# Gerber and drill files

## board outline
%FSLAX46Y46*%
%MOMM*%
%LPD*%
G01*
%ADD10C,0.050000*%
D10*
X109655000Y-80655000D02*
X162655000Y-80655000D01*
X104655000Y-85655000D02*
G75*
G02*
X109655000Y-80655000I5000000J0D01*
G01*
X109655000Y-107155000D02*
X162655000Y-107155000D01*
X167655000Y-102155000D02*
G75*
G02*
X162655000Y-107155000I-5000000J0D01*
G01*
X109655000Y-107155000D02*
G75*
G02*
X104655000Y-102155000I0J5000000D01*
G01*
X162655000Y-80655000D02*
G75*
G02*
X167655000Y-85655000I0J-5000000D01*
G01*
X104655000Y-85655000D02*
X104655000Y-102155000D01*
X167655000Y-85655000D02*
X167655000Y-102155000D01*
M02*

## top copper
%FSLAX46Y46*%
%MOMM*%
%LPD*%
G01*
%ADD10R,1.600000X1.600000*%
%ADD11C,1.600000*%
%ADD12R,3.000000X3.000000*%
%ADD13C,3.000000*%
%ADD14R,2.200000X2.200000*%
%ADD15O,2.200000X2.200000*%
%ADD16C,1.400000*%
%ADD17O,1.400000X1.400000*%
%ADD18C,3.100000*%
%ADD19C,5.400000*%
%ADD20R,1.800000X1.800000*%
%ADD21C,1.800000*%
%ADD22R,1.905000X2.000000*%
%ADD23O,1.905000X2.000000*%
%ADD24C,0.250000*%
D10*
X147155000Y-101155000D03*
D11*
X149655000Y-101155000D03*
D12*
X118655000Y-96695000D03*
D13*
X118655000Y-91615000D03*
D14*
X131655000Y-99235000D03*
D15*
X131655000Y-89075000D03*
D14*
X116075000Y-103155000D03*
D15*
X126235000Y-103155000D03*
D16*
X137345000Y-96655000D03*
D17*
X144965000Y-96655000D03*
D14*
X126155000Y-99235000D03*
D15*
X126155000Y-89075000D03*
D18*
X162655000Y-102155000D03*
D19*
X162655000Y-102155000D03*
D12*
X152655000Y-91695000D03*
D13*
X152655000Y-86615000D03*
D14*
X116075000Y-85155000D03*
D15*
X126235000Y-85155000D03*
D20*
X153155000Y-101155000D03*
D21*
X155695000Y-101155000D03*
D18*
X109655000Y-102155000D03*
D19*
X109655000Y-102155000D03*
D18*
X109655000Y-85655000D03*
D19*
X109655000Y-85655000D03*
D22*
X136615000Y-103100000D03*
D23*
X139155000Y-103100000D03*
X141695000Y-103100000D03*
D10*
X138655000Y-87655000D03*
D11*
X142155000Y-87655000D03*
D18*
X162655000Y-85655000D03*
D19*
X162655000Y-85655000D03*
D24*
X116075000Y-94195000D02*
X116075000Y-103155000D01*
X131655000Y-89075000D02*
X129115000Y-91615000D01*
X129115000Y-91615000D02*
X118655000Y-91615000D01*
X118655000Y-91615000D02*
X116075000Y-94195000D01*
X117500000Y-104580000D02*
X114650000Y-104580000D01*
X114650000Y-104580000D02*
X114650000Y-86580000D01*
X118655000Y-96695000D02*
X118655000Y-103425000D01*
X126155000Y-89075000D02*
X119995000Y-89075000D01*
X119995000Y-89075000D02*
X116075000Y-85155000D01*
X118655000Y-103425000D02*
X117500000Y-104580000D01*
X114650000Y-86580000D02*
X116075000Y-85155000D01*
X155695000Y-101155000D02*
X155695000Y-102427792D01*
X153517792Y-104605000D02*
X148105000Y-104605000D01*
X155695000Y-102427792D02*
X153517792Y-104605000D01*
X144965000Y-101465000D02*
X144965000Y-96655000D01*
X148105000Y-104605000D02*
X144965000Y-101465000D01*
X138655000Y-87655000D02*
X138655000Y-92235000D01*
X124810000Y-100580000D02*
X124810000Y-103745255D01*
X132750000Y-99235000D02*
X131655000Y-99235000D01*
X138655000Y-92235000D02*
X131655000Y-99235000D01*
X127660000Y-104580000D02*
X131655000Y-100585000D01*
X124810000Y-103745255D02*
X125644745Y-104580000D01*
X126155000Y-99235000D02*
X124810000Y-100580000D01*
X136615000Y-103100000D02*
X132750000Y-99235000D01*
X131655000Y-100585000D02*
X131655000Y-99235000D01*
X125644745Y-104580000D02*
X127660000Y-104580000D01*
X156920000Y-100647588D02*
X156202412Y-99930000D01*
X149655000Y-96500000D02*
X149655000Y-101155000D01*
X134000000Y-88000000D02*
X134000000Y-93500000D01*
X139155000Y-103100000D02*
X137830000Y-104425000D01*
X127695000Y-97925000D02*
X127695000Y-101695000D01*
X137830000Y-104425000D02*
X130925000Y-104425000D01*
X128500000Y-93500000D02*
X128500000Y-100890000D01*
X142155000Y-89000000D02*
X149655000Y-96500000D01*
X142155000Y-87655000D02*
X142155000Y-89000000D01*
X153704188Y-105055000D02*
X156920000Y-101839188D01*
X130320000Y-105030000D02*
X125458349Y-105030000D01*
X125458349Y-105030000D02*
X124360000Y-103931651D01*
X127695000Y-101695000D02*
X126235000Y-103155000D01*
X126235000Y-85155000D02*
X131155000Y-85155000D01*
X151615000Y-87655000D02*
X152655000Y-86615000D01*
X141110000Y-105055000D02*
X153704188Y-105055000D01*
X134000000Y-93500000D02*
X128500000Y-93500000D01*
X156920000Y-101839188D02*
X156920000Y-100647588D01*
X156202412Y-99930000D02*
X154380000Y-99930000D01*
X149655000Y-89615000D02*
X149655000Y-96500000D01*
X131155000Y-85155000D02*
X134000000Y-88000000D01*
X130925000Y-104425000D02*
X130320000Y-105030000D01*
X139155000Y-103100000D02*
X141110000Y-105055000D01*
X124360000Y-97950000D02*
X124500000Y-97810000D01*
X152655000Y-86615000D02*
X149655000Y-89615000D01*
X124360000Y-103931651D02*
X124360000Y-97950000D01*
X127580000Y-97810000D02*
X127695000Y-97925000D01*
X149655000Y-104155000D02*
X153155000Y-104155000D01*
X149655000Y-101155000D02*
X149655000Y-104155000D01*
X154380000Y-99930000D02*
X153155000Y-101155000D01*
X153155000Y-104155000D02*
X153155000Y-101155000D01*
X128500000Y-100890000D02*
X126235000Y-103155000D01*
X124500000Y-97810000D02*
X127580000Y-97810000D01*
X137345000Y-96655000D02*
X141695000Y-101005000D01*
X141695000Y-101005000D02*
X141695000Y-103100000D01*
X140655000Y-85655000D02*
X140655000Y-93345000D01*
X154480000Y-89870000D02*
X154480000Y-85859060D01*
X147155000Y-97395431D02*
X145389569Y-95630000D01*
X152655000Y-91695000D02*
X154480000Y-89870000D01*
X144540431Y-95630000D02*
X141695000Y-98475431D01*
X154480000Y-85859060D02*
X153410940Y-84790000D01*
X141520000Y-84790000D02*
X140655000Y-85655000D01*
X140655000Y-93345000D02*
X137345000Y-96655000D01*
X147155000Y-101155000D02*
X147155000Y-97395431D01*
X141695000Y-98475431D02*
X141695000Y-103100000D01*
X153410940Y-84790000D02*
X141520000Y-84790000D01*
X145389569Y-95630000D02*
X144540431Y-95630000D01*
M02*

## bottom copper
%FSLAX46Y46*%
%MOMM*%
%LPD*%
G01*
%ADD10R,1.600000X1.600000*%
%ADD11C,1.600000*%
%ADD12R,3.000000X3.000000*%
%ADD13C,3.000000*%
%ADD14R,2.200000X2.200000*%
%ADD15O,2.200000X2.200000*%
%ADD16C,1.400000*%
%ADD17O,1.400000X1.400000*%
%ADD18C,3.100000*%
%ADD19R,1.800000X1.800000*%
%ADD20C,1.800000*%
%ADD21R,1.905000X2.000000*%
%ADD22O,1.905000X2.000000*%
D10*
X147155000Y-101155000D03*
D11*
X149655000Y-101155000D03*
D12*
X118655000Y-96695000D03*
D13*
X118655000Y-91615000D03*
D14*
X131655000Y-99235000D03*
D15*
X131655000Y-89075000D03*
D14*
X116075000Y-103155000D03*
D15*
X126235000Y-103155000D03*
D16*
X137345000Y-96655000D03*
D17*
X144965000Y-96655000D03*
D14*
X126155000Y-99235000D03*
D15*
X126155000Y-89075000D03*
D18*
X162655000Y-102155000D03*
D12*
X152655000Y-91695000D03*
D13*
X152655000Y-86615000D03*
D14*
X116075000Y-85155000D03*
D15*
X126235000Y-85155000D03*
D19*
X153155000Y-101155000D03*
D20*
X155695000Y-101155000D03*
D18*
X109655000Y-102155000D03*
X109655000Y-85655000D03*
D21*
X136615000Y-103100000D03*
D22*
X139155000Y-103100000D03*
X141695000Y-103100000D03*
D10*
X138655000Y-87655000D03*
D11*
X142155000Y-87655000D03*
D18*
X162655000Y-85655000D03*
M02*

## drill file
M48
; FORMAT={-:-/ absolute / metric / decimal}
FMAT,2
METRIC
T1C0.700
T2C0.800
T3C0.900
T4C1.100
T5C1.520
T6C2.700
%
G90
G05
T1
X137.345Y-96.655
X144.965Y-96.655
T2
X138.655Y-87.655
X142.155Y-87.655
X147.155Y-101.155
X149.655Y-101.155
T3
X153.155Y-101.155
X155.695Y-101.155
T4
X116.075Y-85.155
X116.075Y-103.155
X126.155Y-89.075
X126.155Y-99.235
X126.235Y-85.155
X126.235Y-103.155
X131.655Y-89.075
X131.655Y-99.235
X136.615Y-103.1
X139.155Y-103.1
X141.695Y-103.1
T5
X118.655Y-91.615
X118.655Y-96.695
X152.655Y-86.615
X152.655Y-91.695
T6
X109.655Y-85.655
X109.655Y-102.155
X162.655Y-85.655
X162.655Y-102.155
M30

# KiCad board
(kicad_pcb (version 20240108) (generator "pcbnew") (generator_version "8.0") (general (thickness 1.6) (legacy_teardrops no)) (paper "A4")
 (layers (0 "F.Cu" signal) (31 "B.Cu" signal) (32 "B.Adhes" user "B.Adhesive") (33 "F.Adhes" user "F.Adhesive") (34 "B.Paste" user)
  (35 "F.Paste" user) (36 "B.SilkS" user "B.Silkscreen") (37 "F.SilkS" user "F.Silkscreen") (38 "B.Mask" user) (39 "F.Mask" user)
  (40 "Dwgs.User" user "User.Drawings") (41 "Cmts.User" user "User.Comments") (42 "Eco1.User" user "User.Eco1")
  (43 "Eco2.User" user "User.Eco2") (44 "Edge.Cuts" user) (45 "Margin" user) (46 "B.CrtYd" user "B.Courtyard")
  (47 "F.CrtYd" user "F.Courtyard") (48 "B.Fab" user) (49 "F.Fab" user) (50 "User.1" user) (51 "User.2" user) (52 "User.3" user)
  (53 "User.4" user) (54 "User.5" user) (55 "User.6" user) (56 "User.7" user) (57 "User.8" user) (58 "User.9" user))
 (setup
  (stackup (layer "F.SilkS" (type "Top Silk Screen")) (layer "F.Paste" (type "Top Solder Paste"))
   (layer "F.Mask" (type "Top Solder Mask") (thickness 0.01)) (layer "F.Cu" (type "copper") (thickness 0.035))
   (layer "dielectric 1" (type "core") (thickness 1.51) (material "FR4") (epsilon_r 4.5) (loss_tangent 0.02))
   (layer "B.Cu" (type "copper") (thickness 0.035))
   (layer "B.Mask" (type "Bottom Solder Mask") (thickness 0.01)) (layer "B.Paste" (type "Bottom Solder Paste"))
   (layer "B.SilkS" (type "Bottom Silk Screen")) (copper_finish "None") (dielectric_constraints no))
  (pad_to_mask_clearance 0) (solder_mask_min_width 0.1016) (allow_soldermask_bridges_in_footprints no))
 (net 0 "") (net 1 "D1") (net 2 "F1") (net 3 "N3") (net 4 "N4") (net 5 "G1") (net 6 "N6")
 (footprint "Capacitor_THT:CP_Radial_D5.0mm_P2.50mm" (layer "F.Cu") (at 147.155 101.155)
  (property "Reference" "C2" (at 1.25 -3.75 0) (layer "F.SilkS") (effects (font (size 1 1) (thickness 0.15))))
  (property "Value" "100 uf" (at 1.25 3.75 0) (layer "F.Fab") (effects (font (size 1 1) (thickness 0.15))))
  (pad "1" thru_hole rect (at 0 0) (size 1.6 1.6) (drill 0.8) (layers "*.Cu" "*.Mask") (remove_unused_layers no) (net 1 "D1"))
  (pad "2" thru_hole circle (at 2.5 0) (size 1.6 1.6) (drill 0.8) (layers "*.Cu" "*.Mask") (remove_unused_layers no) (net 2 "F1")))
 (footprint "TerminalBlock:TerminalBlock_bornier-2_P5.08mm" (layer "F.Cu") (at 118.655 96.695 90)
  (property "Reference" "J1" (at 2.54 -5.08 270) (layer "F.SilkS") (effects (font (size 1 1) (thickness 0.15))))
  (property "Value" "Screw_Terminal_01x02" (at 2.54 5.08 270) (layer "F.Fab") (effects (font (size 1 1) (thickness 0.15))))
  (pad "1" thru_hole rect (at 0 0 90) (size 3 3) (drill 1.52) (layers "*.Cu" "*.Mask") (remove_unused_layers no) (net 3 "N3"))
  (pad "2" thru_hole circle (at 5.08 0 90) (size 3 3) (drill 1.52) (layers "*.Cu" "*.Mask") (remove_unused_layers no) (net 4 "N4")))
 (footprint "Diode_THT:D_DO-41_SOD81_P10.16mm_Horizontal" (layer "F.Cu") (at 131.655 99.235 90)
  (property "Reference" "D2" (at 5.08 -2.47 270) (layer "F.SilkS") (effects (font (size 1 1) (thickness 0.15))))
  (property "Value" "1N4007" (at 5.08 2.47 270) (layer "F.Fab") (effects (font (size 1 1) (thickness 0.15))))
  (pad "1" thru_hole rect (at 0 0 90) (size 2.2 2.2) (drill 1.1) (layers "*.Cu" "*.Mask") (remove_unused_layers no) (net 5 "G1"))
  (pad "2" thru_hole oval (at 10.16 0 90) (size 2.2 2.2) (drill 1.1) (layers "*.Cu" "*.Mask") (remove_unused_layers no) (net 4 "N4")))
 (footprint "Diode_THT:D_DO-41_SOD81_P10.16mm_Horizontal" (layer "F.Cu") (at 116.075 103.155)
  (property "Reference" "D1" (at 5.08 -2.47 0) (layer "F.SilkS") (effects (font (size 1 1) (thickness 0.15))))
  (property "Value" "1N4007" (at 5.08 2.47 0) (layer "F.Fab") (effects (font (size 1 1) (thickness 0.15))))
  (pad "1" thru_hole rect (at 0 0) (size 2.2 2.2) (drill 1.1) (layers "*.Cu" "*.Mask") (remove_unused_layers no) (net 4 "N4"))
  (pad "2" thru_hole oval (at 10.16 0) (size 2.2 2.2) (drill 1.1) (layers "*.Cu" "*.Mask") (remove_unused_layers no) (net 2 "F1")))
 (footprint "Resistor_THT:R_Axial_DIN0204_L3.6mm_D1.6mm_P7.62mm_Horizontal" (layer "F.Cu") (at 137.345 96.655)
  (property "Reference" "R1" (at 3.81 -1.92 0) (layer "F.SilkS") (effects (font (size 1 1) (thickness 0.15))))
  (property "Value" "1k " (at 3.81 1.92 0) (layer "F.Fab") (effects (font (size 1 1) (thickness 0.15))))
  (pad "1" thru_hole circle (at 0 0) (size 1.4 1.4) (drill 0.7) (layers "*.Cu" "*.Mask") (remove_unused_layers no) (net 1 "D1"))
  (pad "2" thru_hole oval (at 7.62 0) (size 1.4 1.4) (drill 0.7) (layers "*.Cu" "*.Mask") (remove_unused_layers no) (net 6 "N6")))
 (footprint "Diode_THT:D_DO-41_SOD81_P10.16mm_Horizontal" (layer "F.Cu") (at 126.155 99.235 90)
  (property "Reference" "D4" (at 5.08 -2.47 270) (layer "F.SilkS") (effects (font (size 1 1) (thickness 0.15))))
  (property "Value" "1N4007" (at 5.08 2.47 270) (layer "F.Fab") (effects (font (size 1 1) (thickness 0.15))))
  (pad "1" thru_hole rect (at 0 0 90) (size 2.2 2.2) (drill 1.1) (layers "*.Cu" "*.Mask") (remove_unused_layers no) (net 5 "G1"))
  (pad "2" thru_hole oval (at 10.16 0 90) (size 2.2 2.2) (drill 1.1) (layers "*.Cu" "*.Mask") (remove_unused_layers no) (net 3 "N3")))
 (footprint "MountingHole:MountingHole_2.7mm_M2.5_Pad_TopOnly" (layer "F.Cu") (at 162.655 102.155)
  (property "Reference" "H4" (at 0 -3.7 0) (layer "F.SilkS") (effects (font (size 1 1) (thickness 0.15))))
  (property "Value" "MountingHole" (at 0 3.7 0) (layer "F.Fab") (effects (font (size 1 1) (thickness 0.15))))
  (pad "1" thru_hole circle (at 0 0) (size 3.1 3.1) (drill 2.7) (layers "*.Cu" "*.Mask") (remove_unused_layers no))
  (pad "1" connect circle (at 0 0) (size 5.4 5.4) (layers "F.Cu" "F.Mask")))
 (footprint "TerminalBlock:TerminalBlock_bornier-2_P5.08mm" (layer "F.Cu") (at 152.655 91.695 90)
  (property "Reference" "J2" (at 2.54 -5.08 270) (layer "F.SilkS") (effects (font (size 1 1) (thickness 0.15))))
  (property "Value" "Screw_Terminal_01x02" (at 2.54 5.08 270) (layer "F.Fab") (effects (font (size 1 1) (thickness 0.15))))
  (pad "1" thru_hole rect (at 0 0 90) (size 3 3) (drill 1.52) (layers "*.Cu" "*.Mask") (remove_unused_layers no) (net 1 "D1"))
  (pad "2" thru_hole circle (at 5.08 0 90) (size 3 3) (drill 1.52) (layers "*.Cu" "*.Mask") (remove_unused_layers no) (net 2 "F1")))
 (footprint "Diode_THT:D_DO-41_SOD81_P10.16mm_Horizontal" (layer "F.Cu") (at 116.075 85.155)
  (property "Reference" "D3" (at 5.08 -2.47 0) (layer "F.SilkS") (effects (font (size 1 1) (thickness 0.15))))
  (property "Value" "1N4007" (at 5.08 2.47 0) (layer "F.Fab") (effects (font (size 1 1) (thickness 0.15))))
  (pad "1" thru_hole rect (at 0 0) (size 2.2 2.2) (drill 1.1) (layers "*.Cu" "*.Mask") (remove_unused_layers no) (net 3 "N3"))
  (pad "2" thru_hole oval (at 10.16 0) (size 2.2 2.2) (drill 1.1) (layers "*.Cu" "*.Mask") (remove_unused_layers no) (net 2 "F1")))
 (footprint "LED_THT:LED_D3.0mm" (layer "F.Cu") (at 153.155 101.155)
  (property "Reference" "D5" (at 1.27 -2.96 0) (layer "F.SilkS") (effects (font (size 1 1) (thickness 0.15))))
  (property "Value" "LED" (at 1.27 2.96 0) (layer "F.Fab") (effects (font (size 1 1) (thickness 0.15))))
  (pad "1" thru_hole rect (at 0 0) (size 1.8 1.8) (drill 0.9) (layers "*.Cu" "*.Mask") (remove_unused_layers no) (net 2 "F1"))
  (pad "2" thru_hole circle (at 2.54 0) (size 1.8 1.8) (drill 0.9) (layers "*.Cu" "*.Mask") (remove_unused_layers no) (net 6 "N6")))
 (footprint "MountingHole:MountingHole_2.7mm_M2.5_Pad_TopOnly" (layer "F.Cu") (at 109.655 102.155)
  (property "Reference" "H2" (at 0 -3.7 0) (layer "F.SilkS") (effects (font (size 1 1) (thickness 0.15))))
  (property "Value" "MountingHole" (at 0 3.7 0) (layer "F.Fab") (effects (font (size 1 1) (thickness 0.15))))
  (pad "1" thru_hole circle (at 0 0) (size 3.1 3.1) (drill 2.7) (layers "*.Cu" "*.Mask") (remove_unused_layers no))
  (pad "1" connect circle (at 0 0) (size 5.4 5.4) (layers "F.Cu" "F.Mask")))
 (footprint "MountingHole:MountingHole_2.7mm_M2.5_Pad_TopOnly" (layer "F.Cu") (at 109.655 85.655)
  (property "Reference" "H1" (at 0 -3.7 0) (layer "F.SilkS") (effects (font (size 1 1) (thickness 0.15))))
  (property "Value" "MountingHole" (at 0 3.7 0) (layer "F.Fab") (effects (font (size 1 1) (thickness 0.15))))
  (pad "1" thru_hole circle (at 0 0) (size 3.1 3.1) (drill 2.7) (layers "*.Cu" "*.Mask") (remove_unused_layers no))
  (pad "1" connect circle (at 0 0) (size 5.4 5.4) (layers "F.Cu" "F.Mask")))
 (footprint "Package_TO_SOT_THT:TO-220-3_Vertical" (layer "F.Cu") (at 136.615 103.1)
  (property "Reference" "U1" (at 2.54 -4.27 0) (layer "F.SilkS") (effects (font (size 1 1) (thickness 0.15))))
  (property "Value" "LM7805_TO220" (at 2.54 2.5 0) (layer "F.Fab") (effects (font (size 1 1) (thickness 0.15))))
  (pad "1" thru_hole rect (at 0 0) (size 1.905 2) (drill 1.1) (layers "*.Cu" "*.Mask") (remove_unused_layers no) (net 5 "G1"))
  (pad "2" thru_hole oval (at 2.54 0) (size 1.905 2) (drill 1.1) (layers "*.Cu" "*.Mask") (remove_unused_layers no) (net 2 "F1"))
  (pad "3" thru_hole oval (at 5.08 0) (size 1.905 2) (drill 1.1) (layers "*.Cu" "*.Mask") (remove_unused_layers no) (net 1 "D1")))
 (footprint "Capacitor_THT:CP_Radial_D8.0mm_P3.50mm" (layer "F.Cu") (at 138.655 87.655)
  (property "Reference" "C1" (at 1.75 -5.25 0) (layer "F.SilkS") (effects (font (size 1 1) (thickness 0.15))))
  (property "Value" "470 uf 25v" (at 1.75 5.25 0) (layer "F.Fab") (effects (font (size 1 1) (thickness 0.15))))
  (pad "1" thru_hole rect (at 0 0) (size 1.6 1.6) (drill 0.8) (layers "*.Cu" "*.Mask") (remove_unused_layers no) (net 5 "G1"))
  (pad "2" thru_hole circle (at 3.5 0) (size 1.6 1.6) (drill 0.8) (layers "*.Cu" "*.Mask") (remove_unused_layers no) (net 2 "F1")))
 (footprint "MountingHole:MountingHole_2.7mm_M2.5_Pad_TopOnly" (layer "F.Cu") (at 162.655 85.655)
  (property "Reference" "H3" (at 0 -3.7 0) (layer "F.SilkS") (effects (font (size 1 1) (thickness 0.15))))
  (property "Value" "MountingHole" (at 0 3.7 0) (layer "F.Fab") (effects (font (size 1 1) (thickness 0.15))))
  (pad "1" thru_hole circle (at 0 0) (size 3.1 3.1) (drill 2.7) (layers "*.Cu" "*.Mask") (remove_unused_layers no))
  (pad "1" connect circle (at 0 0) (size 5.4 5.4) (layers "F.Cu" "F.Mask")))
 (gr_line (start 109.655 80.655) (end 162.655 80.655) (stroke (width 0.05) (type default)) (layer "Edge.Cuts"))
 (gr_arc (start 104.655 85.655) (mid 106.119466 82.119466) (end 109.655 80.655) (stroke (width 0.05) (type default)) (layer "Edge.Cuts"))
 (gr_line (start 109.655 107.155) (end 162.655 107.155) (stroke (width 0.05) (type default)) (layer "Edge.Cuts"))
 (gr_arc (start 167.655 102.155) (mid 166.190534 105.690534) (end 162.655 107.155) (stroke (width 0.05) (type default)) (layer "Edge.Cuts"))
 (gr_arc (start 109.655 107.155) (mid 106.119466 105.690534) (end 104.655 102.155) (stroke (width 0.05) (type default)) (layer "Edge.Cuts"))
 (gr_arc (start 162.655 80.655) (mid 166.190534 82.119466) (end 167.655 85.655) (stroke (width 0.05) (type default)) (layer "Edge.Cuts"))
 (gr_line (start 104.655 85.655) (end 104.655 102.155) (stroke (width 0.05) (type default)) (layer "Edge.Cuts"))
 (gr_line (start 167.655 85.655) (end 167.655 102.155) (stroke (width 0.05) (type default)) (layer "Edge.Cuts"))
 (segment (start 116.075 94.195) (end 116.075 103.155) (width 0.25) (layer "F.Cu") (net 4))
 (segment (start 131.655 89.075) (end 129.115 91.615) (width 0.25) (layer "F.Cu") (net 4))
 (segment (start 129.115 91.615) (end 118.655 91.615) (width 0.25) (layer "F.Cu") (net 4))
 (segment (start 118.655 91.615) (end 116.075 94.195) (width 0.25) (layer "F.Cu") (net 4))
 (segment (start 117.5 104.58) (end 114.65 104.58) (width 0.25) (layer "F.Cu") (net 3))
 (segment (start 114.65 104.58) (end 114.65 86.58) (width 0.25) (layer "F.Cu") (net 3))
 (segment (start 118.655 96.695) (end 118.655 103.425) (width 0.25) (layer "F.Cu") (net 3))
 (segment (start 126.155 89.075) (end 119.995 89.075) (width 0.25) (layer "F.Cu") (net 3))
 (segment (start 119.995 89.075) (end 116.075 85.155) (width 0.25) (layer "F.Cu") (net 3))
 (segment (start 118.655 103.425) (end 117.5 104.58) (width 0.25) (layer "F.Cu") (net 3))
 (segment (start 114.65 86.58) (end 116.075 85.155) (width 0.25) (layer "F.Cu") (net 3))
 (segment (start 155.695 101.155) (end 155.695 102.427792) (width 0.25) (layer "F.Cu") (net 6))
 (segment (start 153.517792 104.605) (end 148.105 104.605) (width 0.25) (layer "F.Cu") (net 6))
 (segment (start 155.695 102.427792) (end 153.517792 104.605) (width 0.25) (layer "F.Cu") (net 6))
 (segment (start 144.965 101.465) (end 144.965 96.655) (width 0.25) (layer "F.Cu") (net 6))
 (segment (start 148.105 104.605) (end 144.965 101.465) (width 0.25) (layer "F.Cu") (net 6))
 (segment (start 138.655 87.655) (end 138.655 92.235) (width 0.25) (layer "F.Cu") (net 5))
 (segment (start 124.81 100.58) (end 124.81 103.745255) (width 0.25) (layer "F.Cu") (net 5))
 (segment (start 132.75 99.235) (end 131.655 99.235) (width 0.25) (layer "F.Cu") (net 5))
 (segment (start 138.655 92.235) (end 131.655 99.235) (width 0.25) (layer "F.Cu") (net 5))
 (segment (start 127.66 104.58) (end 131.655 100.585) (width 0.25) (layer "F.Cu") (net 5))
 (segment (start 124.81 103.745255) (end 125.644745 104.58) (width 0.25) (layer "F.Cu") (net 5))
 (segment (start 126.155 99.235) (end 124.81 100.58) (width 0.25) (layer "F.Cu") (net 5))
 (segment (start 136.615 103.1) (end 132.75 99.235) (width 0.25) (layer "F.Cu") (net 5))
 (segment (start 131.655 100.585) (end 131.655 99.235) (width 0.25) (layer "F.Cu") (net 5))
 (segment (start 125.644745 104.58) (end 127.66 104.58) (width 0.25) (layer "F.Cu") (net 5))
 (segment (start 156.92 100.647588) (end 156.202412 99.93) (width 0.25) (layer "F.Cu") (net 2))
 (segment (start 149.655 96.5) (end 149.655 101.155) (width 0.25) (layer "F.Cu") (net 2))
 (segment (start 134 88) (end 134 93.5) (width 0.25) (layer "F.Cu") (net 2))
 (segment (start 139.155 103.1) (end 137.83 104.425) (width 0.25) (layer "F.Cu") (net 2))
 (segment (start 127.695 97.925) (end 127.695 101.695) (width 0.25) (layer "F.Cu") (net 2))
 (segment (start 137.83 104.425) (end 130.925 104.425) (width 0.25) (layer "F.Cu") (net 2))
 (segment (start 128.5 93.5) (end 128.5 100.89) (width 0.25) (layer "F.Cu") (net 2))
 (segment (start 142.155 89) (end 149.655 96.5) (width 0.25) (layer "F.Cu") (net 2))
 (segment (start 142.155 87.655) (end 142.155 89) (width 0.25) (layer "F.Cu") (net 2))
 (segment (start 153.704188 105.055) (end 156.92 101.839188) (width 0.25) (layer "F.Cu") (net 2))
 (segment (start 130.32 105.03) (end 125.458349 105.03) (width 0.25) (layer "F.Cu") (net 2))
 (segment (start 125.458349 105.03) (end 124.36 103.931651) (width 0.25) (layer "F.Cu") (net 2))
 (segment (start 127.695 101.695) (end 126.235 103.155) (width 0.25) (layer "F.Cu") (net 2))
 (segment (start 126.235 85.155) (end 131.155 85.155) (width 0.25) (layer "F.Cu") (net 2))
 (segment (start 151.615 87.655) (end 152.655 86.615) (width 0.25) (layer "F.Cu") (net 2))
 (segment (start 141.11 105.055) (end 153.704188 105.055) (width 0.25) (layer "F.Cu") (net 2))
 (segment (start 134 93.5) (end 128.5 93.5) (width 0.25) (layer "F.Cu") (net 2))
 (segment (start 156.92 101.839188) (end 156.92 100.647588) (width 0.25) (layer "F.Cu") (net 2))
 (segment (start 156.202412 99.93) (end 154.38 99.93) (width 0.25) (layer "F.Cu") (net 2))
 (segment (start 149.655 89.615) (end 149.655 96.5) (width 0.25) (layer "F.Cu") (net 2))
 (segment (start 131.155 85.155) (end 134 88) (width 0.25) (layer "F.Cu") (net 2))
 (segment (start 130.925 104.425) (end 130.32 105.03) (width 0.25) (layer "F.Cu") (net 2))
 (segment (start 139.155 103.1) (end 141.11 105.055) (width 0.25) (layer "F.Cu") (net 2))
 (segment (start 124.36 97.95) (end 124.5 97.81) (width 0.25) (layer "F.Cu") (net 2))
 (segment (start 152.655 86.615) (end 149.655 89.615) (width 0.25) (layer "F.Cu") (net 2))
 (segment (start 124.36 103.931651) (end 124.36 97.95) (width 0.25) (layer "F.Cu") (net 2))
 (segment (start 127.58 97.81) (end 127.695 97.925) (width 0.25) (layer "F.Cu") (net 2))
 (segment (start 149.655 104.155) (end 153.155 104.155) (width 0.25) (layer "F.Cu") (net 2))
 (segment (start 149.655 101.155) (end 149.655 104.155) (width 0.25) (layer "F.Cu") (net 2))
 (segment (start 154.38 99.93) (end 153.155 101.155) (width 0.25) (layer "F.Cu") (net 2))
 (segment (start 153.155 104.155) (end 153.155 101.155) (width 0.25) (layer "F.Cu") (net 2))
 (segment (start 128.5 100.89) (end 126.235 103.155) (width 0.25) (layer "F.Cu") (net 2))
 (segment (start 124.5 97.81) (end 127.58 97.81) (width 0.25) (layer "F.Cu") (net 2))
 (segment (start 137.345 96.655) (end 141.695 101.005) (width 0.25) (layer "F.Cu") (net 1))
 (segment (start 141.695 101.005) (end 141.695 103.1) (width 0.25) (layer "F.Cu") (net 1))
 (segment (start 140.655 85.655) (end 140.655 93.345) (width 0.25) (layer "F.Cu") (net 1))
 (segment (start 154.48 89.87) (end 154.48 85.85906) (width 0.25) (layer "F.Cu") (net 1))
 (segment (start 147.155 97.395431) (end 145.389569 95.63) (width 0.25) (layer "F.Cu") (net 1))
 (segment (start 152.655 91.695) (end 154.48 89.87) (width 0.25) (layer "F.Cu") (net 1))
 (segment (start 144.540431 95.63) (end 141.695 98.475431) (width 0.25) (layer "F.Cu") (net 1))
 (segment (start 154.48 85.85906) (end 153.41094 84.79) (width 0.25) (layer "F.Cu") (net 1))
 (segment (start 141.52 84.79) (end 140.655 85.655) (width 0.25) (layer "F.Cu") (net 1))
 (segment (start 140.655 93.345) (end 137.345 96.655) (width 0.25) (layer "F.Cu") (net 1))
 (segment (start 147.155 101.155) (end 147.155 97.395431) (width 0.25) (layer "F.Cu") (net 1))
 (segment (start 141.695 98.475431) (end 141.695 103.1) (width 0.25) (layer "F.Cu") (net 1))
 (segment (start 153.41094 84.79) (end 141.52 84.79) (width 0.25) (layer "F.Cu") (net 1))
 (segment (start 145.389569 95.63) (end 144.540431 95.63) (width 0.25) (layer "F.Cu") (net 1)))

